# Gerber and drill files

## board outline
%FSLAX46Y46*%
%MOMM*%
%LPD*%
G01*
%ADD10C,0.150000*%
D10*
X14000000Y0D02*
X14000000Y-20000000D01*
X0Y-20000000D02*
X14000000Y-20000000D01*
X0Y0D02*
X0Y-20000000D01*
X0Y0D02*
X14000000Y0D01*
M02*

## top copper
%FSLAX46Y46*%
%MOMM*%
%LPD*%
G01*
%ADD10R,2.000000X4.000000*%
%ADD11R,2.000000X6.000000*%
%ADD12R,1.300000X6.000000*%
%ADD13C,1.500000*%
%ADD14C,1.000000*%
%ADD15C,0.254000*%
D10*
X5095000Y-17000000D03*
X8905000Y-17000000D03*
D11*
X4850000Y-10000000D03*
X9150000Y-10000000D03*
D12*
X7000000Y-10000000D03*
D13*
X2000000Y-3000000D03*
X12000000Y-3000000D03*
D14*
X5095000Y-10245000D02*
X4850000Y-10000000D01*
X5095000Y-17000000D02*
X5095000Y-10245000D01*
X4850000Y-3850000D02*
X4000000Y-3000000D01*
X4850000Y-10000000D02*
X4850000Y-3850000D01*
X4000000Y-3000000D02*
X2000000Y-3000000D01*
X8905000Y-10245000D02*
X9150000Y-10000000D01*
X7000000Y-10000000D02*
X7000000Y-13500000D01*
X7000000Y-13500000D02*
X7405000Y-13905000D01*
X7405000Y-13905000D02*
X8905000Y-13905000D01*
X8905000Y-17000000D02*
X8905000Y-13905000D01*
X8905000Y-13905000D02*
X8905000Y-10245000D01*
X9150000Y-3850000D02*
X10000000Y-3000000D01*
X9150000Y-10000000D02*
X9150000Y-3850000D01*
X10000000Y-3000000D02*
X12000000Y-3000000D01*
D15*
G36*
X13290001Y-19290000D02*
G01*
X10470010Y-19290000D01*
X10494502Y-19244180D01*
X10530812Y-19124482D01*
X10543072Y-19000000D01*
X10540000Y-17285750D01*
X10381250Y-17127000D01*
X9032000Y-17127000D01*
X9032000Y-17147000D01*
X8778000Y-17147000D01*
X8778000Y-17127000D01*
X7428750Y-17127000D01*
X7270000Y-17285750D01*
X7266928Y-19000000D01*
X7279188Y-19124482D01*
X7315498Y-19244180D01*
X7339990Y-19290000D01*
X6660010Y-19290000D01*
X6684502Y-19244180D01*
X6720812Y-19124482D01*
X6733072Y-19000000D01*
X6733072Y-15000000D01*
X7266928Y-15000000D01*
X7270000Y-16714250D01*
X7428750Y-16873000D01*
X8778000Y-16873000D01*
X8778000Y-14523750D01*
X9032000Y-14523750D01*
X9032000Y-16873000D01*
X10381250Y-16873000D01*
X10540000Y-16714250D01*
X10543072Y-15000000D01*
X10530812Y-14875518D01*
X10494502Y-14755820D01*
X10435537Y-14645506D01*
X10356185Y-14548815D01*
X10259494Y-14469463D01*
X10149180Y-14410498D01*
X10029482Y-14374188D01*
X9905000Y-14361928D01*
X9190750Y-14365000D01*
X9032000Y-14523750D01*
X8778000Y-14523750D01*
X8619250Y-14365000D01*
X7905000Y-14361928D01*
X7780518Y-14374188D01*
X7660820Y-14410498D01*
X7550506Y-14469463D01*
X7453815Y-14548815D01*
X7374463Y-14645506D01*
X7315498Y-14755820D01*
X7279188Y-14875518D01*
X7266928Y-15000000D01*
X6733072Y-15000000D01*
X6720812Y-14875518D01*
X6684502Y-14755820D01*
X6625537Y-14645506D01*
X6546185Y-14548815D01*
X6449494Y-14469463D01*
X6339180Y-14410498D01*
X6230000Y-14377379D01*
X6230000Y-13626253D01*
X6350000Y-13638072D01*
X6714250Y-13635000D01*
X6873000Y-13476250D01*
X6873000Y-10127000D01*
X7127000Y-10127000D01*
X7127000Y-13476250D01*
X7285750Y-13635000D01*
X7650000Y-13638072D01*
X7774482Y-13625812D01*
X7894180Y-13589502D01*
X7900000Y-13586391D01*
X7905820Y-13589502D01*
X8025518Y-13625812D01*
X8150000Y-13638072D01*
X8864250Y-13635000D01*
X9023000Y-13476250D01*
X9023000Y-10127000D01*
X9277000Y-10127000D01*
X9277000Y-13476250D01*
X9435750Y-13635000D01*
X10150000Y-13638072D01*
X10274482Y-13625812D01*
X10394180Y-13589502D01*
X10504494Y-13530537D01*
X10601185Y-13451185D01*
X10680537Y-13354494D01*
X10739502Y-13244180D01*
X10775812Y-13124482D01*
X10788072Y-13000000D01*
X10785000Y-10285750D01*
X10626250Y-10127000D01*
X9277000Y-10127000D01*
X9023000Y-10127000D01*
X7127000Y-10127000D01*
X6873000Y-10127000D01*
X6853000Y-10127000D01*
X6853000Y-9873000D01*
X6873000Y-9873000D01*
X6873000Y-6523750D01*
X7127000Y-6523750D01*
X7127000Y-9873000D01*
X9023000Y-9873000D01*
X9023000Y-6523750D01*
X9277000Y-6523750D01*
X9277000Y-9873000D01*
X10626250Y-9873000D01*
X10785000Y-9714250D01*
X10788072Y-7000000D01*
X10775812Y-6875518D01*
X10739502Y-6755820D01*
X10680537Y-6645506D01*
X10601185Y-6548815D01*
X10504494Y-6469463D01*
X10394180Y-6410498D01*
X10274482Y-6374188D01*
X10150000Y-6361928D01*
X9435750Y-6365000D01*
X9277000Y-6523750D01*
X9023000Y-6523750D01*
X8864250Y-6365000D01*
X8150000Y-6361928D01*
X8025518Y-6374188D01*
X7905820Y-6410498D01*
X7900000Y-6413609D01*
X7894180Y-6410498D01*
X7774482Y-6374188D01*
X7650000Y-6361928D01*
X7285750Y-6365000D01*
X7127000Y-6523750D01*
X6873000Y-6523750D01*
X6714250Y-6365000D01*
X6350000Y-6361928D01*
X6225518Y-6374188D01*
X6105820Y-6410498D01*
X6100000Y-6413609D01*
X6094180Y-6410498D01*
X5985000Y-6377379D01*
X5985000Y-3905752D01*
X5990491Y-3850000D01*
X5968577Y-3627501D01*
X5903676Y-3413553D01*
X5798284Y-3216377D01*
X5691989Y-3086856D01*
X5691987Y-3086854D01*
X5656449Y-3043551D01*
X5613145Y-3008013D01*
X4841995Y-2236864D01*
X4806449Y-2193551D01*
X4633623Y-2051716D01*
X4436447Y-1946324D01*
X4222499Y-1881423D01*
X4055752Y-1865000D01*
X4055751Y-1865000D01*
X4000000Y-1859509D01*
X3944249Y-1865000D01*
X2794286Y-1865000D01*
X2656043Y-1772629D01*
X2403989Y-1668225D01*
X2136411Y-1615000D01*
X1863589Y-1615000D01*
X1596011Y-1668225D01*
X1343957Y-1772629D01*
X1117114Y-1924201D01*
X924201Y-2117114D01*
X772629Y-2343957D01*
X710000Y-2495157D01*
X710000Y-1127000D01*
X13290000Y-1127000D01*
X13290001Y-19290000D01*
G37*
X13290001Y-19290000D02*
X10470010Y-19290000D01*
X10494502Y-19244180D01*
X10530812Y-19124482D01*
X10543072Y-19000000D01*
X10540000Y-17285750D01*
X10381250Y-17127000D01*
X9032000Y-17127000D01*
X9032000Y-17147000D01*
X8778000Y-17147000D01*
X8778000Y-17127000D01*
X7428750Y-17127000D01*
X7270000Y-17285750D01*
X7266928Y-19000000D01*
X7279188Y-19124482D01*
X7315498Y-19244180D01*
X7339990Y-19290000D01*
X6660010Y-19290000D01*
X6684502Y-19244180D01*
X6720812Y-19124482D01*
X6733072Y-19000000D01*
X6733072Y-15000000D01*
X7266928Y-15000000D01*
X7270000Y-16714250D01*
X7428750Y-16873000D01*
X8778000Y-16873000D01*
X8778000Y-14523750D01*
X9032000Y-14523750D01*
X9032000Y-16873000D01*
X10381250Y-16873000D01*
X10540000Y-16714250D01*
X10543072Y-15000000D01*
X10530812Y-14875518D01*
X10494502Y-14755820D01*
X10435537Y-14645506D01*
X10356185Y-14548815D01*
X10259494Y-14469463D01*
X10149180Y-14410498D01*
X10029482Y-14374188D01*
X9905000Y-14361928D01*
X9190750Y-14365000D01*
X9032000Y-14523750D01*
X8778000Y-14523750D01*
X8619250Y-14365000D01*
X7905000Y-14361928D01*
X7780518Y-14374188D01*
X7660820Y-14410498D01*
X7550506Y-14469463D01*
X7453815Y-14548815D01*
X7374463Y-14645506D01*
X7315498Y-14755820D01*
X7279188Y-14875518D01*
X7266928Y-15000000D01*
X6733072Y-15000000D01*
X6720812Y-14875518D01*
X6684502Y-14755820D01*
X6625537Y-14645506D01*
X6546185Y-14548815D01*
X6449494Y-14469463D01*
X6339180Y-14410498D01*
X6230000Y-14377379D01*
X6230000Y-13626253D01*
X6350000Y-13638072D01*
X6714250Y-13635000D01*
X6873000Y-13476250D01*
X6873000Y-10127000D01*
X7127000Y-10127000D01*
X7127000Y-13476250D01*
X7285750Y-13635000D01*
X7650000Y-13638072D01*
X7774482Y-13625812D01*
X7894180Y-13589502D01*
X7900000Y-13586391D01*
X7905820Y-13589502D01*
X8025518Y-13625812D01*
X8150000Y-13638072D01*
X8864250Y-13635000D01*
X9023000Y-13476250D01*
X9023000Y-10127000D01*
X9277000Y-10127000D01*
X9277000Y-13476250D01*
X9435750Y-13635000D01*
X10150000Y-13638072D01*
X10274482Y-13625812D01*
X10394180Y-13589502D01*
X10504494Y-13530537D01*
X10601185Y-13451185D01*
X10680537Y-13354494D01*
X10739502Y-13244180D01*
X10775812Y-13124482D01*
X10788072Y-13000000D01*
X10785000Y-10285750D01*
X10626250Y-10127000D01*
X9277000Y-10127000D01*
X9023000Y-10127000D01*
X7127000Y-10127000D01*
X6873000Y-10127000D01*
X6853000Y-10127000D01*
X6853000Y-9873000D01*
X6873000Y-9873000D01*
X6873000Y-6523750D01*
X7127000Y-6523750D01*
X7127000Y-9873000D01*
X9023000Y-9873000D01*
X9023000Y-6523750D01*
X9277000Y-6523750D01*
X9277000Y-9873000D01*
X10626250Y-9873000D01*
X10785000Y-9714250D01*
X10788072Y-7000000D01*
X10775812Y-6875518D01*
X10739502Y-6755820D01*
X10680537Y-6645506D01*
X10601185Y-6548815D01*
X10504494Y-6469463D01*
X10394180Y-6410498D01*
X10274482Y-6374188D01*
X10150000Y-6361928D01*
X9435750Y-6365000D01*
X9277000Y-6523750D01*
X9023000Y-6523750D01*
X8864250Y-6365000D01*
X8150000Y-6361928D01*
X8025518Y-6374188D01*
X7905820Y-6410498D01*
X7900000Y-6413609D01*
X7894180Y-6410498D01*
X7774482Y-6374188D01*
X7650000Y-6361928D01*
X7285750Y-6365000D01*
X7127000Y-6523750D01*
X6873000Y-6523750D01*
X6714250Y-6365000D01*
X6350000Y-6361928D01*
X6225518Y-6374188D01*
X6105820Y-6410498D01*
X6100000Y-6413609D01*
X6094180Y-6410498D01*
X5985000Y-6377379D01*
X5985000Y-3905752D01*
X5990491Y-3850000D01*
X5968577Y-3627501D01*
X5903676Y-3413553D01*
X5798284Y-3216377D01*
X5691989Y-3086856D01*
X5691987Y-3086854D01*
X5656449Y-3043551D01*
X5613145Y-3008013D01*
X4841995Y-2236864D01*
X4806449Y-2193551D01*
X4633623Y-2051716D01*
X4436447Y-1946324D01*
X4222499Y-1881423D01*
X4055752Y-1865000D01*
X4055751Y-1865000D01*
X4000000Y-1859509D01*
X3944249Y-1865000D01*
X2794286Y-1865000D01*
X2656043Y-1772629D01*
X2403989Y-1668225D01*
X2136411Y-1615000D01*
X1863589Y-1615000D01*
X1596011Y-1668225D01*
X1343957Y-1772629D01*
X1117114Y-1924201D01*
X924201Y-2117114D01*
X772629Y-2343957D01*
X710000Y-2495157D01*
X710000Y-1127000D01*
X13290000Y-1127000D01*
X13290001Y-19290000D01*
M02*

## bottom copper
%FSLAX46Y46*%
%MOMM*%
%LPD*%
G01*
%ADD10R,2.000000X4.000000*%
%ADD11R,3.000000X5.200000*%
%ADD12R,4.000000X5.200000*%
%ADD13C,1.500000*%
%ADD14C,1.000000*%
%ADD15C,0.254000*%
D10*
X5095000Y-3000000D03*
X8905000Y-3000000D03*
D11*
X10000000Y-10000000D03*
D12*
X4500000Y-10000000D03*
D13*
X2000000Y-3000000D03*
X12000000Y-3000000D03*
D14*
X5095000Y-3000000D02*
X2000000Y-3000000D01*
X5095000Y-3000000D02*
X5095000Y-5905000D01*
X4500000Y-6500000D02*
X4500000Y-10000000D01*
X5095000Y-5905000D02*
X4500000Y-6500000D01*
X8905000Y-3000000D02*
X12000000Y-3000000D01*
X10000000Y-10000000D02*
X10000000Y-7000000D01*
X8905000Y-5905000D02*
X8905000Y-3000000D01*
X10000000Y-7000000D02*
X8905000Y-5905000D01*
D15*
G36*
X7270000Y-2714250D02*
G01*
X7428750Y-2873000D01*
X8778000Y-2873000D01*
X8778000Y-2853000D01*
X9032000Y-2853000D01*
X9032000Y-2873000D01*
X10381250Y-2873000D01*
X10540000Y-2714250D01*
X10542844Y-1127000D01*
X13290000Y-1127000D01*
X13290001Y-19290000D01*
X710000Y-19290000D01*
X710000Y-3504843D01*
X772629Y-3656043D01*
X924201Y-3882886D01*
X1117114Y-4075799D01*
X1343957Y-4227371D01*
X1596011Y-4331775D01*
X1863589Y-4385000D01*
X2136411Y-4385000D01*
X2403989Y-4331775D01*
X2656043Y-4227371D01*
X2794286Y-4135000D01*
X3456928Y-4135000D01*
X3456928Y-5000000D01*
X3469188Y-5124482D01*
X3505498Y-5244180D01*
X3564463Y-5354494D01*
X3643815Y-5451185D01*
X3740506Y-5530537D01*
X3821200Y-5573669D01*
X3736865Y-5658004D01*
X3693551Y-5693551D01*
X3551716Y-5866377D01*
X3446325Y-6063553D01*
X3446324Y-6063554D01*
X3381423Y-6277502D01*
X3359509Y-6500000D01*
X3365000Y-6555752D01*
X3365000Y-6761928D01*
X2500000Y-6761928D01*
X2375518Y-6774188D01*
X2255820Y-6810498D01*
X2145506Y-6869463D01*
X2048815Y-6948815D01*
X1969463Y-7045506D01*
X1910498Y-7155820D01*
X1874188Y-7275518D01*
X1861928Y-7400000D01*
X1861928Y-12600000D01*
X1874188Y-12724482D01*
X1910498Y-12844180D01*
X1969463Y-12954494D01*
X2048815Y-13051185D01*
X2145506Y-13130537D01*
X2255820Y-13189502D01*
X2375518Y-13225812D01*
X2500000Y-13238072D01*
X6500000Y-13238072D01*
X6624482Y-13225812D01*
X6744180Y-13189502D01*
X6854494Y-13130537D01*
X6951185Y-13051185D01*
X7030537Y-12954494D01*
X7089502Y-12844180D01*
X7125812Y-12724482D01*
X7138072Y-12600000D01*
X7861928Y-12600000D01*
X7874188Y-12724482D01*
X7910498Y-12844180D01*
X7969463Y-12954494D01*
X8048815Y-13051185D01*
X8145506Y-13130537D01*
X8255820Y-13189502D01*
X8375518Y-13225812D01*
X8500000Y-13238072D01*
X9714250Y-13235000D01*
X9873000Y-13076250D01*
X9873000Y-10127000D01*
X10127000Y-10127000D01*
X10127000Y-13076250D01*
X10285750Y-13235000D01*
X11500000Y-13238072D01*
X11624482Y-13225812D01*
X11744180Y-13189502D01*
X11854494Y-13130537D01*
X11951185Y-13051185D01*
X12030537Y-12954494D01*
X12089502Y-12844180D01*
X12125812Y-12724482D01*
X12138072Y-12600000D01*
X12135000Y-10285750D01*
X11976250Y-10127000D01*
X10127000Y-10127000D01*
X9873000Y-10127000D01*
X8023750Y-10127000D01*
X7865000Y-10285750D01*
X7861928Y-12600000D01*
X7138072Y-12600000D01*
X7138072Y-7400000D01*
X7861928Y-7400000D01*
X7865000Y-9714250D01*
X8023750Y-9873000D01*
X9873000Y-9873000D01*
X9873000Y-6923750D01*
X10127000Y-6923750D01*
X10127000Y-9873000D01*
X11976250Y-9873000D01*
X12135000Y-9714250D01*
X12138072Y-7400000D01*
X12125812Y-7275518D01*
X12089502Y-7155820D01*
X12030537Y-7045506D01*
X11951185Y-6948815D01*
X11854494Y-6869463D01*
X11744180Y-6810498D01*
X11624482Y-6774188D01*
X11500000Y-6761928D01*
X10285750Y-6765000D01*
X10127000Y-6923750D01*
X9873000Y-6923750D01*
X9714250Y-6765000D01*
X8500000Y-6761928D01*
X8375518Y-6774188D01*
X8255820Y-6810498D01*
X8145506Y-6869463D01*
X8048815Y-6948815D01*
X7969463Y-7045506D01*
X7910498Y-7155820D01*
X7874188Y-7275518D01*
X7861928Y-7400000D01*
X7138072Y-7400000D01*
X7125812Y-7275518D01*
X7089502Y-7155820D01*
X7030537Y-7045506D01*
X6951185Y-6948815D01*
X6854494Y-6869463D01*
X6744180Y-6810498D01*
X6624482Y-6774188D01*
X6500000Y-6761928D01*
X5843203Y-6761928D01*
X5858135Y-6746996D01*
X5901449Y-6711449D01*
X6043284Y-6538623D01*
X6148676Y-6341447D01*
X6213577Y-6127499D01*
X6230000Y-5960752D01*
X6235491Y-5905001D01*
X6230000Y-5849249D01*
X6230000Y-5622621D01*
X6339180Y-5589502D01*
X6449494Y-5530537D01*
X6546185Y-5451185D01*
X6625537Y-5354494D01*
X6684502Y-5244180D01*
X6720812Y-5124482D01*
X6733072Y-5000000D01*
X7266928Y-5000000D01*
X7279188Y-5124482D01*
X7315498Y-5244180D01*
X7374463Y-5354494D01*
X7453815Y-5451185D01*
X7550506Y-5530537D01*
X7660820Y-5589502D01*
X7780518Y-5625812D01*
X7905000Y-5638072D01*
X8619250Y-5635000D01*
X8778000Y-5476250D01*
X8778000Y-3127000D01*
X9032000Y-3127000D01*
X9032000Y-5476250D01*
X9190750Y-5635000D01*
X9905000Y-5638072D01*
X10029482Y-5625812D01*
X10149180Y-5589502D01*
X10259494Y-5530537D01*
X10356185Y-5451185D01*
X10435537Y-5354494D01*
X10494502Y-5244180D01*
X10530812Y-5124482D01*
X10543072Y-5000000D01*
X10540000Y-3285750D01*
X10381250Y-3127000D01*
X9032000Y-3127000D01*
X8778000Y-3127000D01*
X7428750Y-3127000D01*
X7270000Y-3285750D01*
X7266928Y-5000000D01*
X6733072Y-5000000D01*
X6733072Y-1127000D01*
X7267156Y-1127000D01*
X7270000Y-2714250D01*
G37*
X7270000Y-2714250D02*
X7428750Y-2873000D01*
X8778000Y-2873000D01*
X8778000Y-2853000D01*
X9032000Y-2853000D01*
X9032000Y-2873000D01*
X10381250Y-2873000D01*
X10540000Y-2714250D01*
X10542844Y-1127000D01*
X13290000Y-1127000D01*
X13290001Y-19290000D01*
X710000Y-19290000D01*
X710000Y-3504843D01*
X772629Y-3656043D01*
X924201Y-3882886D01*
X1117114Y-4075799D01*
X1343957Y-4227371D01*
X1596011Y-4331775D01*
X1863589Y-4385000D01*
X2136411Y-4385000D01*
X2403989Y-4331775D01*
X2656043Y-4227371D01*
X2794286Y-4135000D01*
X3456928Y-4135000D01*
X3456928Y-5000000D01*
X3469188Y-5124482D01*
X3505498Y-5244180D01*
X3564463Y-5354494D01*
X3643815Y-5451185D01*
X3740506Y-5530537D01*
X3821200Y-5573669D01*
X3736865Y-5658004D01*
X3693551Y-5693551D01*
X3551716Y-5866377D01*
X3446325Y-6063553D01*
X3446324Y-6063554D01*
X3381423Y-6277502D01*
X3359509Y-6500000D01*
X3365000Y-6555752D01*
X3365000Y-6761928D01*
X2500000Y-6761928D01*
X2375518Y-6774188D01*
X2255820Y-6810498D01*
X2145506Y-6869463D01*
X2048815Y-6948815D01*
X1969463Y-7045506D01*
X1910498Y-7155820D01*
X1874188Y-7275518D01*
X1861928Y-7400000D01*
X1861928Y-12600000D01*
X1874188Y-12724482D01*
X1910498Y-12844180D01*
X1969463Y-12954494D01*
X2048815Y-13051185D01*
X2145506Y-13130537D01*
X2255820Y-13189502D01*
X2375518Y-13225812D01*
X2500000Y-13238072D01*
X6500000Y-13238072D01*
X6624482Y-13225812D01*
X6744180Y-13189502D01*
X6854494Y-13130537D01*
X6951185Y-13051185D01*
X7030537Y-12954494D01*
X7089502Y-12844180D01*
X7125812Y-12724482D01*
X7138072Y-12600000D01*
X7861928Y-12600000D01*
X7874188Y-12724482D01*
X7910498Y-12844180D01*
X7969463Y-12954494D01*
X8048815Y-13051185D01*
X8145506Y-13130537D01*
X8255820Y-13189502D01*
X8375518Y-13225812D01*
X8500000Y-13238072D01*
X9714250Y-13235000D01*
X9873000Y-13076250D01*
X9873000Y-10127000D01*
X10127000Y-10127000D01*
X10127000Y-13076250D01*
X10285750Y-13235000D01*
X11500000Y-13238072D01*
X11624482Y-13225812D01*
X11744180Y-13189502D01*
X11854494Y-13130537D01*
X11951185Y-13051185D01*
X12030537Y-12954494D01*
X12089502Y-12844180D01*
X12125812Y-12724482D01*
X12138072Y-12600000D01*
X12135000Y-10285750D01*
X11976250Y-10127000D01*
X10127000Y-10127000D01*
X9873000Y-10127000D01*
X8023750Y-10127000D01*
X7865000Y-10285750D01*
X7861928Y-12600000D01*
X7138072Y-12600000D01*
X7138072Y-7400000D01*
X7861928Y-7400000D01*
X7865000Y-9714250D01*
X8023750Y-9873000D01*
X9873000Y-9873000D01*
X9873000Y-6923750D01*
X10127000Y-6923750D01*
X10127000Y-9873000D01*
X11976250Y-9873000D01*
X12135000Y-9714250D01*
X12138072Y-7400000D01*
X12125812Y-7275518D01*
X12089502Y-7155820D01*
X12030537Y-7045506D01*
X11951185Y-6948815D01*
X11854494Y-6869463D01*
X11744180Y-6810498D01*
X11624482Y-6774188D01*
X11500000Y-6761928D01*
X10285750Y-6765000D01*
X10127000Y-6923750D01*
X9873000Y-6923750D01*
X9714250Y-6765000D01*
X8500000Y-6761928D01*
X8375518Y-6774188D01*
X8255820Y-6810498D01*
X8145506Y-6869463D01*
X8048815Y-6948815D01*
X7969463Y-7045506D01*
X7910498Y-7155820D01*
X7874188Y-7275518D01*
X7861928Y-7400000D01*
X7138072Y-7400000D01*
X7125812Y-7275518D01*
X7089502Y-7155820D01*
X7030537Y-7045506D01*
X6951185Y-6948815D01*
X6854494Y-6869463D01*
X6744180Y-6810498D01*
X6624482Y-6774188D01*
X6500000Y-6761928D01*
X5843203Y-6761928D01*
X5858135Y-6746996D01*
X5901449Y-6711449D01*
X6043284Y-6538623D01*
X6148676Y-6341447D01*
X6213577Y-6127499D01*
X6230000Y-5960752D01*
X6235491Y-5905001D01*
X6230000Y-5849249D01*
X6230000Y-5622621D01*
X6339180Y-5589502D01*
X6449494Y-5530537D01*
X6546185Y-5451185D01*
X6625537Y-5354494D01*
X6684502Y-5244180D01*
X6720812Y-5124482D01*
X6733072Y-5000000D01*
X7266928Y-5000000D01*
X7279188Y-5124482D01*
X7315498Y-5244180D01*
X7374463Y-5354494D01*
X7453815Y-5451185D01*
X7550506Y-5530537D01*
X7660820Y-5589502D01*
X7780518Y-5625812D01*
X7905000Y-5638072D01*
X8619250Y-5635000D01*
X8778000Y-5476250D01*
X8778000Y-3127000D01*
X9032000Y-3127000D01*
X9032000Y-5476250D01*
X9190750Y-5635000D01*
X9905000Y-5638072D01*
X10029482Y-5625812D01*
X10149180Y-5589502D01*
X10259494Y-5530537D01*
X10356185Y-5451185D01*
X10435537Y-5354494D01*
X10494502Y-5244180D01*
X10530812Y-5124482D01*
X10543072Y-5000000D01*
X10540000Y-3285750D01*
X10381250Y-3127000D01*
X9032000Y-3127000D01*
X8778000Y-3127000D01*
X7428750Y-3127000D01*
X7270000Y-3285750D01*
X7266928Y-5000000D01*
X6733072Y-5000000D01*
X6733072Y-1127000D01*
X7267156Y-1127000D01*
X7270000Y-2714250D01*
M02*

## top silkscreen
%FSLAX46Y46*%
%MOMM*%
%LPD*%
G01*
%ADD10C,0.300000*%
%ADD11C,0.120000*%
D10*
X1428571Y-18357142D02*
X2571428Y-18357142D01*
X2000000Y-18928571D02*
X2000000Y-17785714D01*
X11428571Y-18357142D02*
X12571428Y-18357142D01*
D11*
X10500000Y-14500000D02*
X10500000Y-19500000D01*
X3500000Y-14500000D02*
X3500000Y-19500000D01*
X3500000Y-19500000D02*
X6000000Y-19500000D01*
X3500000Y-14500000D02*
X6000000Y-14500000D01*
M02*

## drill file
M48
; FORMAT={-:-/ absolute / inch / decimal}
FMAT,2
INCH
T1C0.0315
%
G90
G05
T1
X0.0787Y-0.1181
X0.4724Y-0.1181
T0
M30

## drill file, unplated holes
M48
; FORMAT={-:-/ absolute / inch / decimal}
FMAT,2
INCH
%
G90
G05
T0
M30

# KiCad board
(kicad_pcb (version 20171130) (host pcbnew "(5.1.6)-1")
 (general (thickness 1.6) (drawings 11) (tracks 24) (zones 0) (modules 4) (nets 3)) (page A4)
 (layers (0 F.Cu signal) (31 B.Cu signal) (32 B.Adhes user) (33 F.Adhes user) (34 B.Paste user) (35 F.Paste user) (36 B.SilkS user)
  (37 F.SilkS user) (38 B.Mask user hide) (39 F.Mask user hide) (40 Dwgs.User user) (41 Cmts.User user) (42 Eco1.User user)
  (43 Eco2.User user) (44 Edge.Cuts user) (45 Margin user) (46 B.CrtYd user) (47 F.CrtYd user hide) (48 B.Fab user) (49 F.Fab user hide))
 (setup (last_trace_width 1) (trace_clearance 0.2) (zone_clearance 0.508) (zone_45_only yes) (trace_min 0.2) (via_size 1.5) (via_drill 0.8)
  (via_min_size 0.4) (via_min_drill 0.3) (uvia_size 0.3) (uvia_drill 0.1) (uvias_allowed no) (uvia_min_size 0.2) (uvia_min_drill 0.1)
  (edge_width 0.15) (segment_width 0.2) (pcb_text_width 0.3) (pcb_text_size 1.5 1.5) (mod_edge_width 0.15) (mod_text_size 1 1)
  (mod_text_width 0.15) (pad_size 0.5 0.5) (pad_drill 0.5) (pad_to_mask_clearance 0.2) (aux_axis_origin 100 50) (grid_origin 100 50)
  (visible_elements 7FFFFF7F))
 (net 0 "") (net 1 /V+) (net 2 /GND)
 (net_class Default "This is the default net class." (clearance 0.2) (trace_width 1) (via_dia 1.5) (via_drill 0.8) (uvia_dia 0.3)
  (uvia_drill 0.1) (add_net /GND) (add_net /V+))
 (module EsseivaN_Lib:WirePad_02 (layer F.Cu) (at 107 67)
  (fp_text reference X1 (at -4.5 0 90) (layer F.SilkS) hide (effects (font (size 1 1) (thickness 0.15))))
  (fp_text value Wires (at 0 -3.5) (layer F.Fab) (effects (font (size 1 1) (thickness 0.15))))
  (fp_line (start -3.5 -2.5) (end -1 -2.5) (layer F.SilkS) (width 0.12))
  (fp_line (start -3.5 2.5) (end -1 2.5) (layer F.SilkS) (width 0.12))
  (fp_line (start -3.5 -2.5) (end -3.5 2.5) (layer F.SilkS) (width 0.12))
  (fp_line (start 3.5 -2.5) (end 3.5 2.5) (layer F.SilkS) (width 0.12))
  (pad 1 connect rect (at -1.905 0) (size 2 4) (layers F.Cu F.Mask) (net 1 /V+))
  (pad 2 connect rect (at 1.905 0) (size 2 4) (layers F.Cu F.Mask) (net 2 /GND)))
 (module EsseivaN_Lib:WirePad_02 (layer B.Cu) (at 107 53)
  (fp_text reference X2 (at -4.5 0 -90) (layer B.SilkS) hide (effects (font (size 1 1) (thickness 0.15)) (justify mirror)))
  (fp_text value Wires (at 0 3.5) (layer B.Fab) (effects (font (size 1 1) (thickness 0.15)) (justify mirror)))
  (pad 1 connect rect (at -1.905 0) (size 2 4) (layers B.Cu B.Mask) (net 1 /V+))
  (pad 2 connect rect (at 1.905 0) (size 2 4) (layers B.Cu B.Mask) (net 2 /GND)))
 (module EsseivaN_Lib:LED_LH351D (layer F.Cu) (at 107 60 90)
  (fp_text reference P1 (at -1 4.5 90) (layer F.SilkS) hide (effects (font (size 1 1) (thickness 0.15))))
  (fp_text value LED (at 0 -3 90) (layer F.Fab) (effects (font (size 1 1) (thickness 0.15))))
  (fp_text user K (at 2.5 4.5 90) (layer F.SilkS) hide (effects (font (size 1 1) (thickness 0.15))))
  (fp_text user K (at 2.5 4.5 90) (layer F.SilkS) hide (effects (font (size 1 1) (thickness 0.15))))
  (pad 2 smd rect (at 0 -2.15 90) (size 6 2) (layers F.Cu F.Paste F.Mask) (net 1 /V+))
  (pad 1 smd rect (at 0 2.15 90) (size 6 2) (layers F.Cu F.Paste F.Mask) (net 2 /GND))
  (pad 1 smd rect (at 0 0 90) (size 6 1.3) (layers F.Cu F.Paste F.Mask) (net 2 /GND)))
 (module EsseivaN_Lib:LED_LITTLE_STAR (layer B.Cu) (at 107 60 90)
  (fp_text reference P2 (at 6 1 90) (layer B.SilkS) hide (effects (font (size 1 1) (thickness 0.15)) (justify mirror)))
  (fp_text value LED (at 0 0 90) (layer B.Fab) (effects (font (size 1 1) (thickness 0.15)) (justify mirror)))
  (pad 1 smd rect (at 0 3 90) (size 5.2 3) (layers B.Cu B.Paste B.Mask) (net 2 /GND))
  (pad 2 smd rect (at 0 -2.5 90) (size 5.2 4) (layers B.Cu B.Paste B.Mask) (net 1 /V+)))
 (gr_line (start 114 50) (end 114 70) (layer Edge.Cuts) (width 0.15))
 (gr_line (start 100 70) (end 114 70) (layer Edge.Cuts) (width 0.15))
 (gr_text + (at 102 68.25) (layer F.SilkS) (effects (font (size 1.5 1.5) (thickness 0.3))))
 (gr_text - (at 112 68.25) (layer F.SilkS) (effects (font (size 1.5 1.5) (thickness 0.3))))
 (gr_line (start 100 50) (end 100 70) (layer Edge.Cuts) (width 0.15))
 (gr_line (start 100 50) (end 114 50) (layer Edge.Cuts) (width 0.15))
 (via (at 102 53) (size 1.5) (drill 0.8) (layers F.Cu B.Cu) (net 1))
 (segment (start 105.095 53) (end 102 53) (width 1) (layer B.Cu) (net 1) (status 10))
 (segment (start 105.095 53) (end 105.095 55.905) (width 1) (layer B.Cu) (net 1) (status 10))
 (segment (start 104.5 56.5) (end 104.5 60) (width 1) (layer B.Cu) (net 1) (status 20))
 (segment (start 105.095 55.905) (end 104.5 56.5) (width 1) (layer B.Cu) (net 1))
 (segment (start 105.095 60.245) (end 104.85 60) (width 1) (layer F.Cu) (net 1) (status 30))
 (segment (start 105.095 67) (end 105.095 60.245) (width 1) (layer F.Cu) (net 1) (status 30))
 (segment (start 104.85 53.85) (end 104 53) (width 1) (layer F.Cu) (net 1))
 (segment (start 104.85 60) (end 104.85 53.85) (width 1) (layer F.Cu) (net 1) (status 10))
 (segment (start 104 53) (end 102 53) (width 1) (layer F.Cu) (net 1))
 (via (at 112 53) (size 1.5) (drill 0.8) (layers F.Cu B.Cu) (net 2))
 (segment (start 108.905 53) (end 112 53) (width 1) (layer B.Cu) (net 2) (status 10))
 (segment (start 110 60) (end 110 57) (width 1) (layer B.Cu) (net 2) (status 10))
 (segment (start 108.905 55.905) (end 108.905 53) (width 1) (layer B.Cu) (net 2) (status 20))
 (segment (start 110 57) (end 108.905 55.905) (width 1) (layer B.Cu) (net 2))
 (segment (start 108.905 60.245) (end 109.15 60) (width 1) (layer F.Cu) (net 2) (status 30))
 (segment (start 107 60) (end 107 63.5) (width 1) (layer F.Cu) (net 2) (status 10))
 (segment (start 107 63.5) (end 107.405 63.905) (width 1) (layer F.Cu) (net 2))
 (segment (start 107.405 63.905) (end 108.905 63.905) (width 1) (layer F.Cu) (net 2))
 (segment (start 108.905 67) (end 108.905 63.905) (width 1) (layer F.Cu) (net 2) (status 10))
 (segment (start 108.905 63.905) (end 108.905 60.245) (width 1) (layer F.Cu) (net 2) (status 20))
 (segment (start 109.15 53.85) (end 110 53) (width 1) (layer F.Cu) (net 2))
 (segment (start 109.15 60) (end 109.15 53.85) (width 1) (layer F.Cu) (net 2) (status 10))
 (segment (start 110 53) (end 112 53) (width 1) (layer F.Cu) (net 2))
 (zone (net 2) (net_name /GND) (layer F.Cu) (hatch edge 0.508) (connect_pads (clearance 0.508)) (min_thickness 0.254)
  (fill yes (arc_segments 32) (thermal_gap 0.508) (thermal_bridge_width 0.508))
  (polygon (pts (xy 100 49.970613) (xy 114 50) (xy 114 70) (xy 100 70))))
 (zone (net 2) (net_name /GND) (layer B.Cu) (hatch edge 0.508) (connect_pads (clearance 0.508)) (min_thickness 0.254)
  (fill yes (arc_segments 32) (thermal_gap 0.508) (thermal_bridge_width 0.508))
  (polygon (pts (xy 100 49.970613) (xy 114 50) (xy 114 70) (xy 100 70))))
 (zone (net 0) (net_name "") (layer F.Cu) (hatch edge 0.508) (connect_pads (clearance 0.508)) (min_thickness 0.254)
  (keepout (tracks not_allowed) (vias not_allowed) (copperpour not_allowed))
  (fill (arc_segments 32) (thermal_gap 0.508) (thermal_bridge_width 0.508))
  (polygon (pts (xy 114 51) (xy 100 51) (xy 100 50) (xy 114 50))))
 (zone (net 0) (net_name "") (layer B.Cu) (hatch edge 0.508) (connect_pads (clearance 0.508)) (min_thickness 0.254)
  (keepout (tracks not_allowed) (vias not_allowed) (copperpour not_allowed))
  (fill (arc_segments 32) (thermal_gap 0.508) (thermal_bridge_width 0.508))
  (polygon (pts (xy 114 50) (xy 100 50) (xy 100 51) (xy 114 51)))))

